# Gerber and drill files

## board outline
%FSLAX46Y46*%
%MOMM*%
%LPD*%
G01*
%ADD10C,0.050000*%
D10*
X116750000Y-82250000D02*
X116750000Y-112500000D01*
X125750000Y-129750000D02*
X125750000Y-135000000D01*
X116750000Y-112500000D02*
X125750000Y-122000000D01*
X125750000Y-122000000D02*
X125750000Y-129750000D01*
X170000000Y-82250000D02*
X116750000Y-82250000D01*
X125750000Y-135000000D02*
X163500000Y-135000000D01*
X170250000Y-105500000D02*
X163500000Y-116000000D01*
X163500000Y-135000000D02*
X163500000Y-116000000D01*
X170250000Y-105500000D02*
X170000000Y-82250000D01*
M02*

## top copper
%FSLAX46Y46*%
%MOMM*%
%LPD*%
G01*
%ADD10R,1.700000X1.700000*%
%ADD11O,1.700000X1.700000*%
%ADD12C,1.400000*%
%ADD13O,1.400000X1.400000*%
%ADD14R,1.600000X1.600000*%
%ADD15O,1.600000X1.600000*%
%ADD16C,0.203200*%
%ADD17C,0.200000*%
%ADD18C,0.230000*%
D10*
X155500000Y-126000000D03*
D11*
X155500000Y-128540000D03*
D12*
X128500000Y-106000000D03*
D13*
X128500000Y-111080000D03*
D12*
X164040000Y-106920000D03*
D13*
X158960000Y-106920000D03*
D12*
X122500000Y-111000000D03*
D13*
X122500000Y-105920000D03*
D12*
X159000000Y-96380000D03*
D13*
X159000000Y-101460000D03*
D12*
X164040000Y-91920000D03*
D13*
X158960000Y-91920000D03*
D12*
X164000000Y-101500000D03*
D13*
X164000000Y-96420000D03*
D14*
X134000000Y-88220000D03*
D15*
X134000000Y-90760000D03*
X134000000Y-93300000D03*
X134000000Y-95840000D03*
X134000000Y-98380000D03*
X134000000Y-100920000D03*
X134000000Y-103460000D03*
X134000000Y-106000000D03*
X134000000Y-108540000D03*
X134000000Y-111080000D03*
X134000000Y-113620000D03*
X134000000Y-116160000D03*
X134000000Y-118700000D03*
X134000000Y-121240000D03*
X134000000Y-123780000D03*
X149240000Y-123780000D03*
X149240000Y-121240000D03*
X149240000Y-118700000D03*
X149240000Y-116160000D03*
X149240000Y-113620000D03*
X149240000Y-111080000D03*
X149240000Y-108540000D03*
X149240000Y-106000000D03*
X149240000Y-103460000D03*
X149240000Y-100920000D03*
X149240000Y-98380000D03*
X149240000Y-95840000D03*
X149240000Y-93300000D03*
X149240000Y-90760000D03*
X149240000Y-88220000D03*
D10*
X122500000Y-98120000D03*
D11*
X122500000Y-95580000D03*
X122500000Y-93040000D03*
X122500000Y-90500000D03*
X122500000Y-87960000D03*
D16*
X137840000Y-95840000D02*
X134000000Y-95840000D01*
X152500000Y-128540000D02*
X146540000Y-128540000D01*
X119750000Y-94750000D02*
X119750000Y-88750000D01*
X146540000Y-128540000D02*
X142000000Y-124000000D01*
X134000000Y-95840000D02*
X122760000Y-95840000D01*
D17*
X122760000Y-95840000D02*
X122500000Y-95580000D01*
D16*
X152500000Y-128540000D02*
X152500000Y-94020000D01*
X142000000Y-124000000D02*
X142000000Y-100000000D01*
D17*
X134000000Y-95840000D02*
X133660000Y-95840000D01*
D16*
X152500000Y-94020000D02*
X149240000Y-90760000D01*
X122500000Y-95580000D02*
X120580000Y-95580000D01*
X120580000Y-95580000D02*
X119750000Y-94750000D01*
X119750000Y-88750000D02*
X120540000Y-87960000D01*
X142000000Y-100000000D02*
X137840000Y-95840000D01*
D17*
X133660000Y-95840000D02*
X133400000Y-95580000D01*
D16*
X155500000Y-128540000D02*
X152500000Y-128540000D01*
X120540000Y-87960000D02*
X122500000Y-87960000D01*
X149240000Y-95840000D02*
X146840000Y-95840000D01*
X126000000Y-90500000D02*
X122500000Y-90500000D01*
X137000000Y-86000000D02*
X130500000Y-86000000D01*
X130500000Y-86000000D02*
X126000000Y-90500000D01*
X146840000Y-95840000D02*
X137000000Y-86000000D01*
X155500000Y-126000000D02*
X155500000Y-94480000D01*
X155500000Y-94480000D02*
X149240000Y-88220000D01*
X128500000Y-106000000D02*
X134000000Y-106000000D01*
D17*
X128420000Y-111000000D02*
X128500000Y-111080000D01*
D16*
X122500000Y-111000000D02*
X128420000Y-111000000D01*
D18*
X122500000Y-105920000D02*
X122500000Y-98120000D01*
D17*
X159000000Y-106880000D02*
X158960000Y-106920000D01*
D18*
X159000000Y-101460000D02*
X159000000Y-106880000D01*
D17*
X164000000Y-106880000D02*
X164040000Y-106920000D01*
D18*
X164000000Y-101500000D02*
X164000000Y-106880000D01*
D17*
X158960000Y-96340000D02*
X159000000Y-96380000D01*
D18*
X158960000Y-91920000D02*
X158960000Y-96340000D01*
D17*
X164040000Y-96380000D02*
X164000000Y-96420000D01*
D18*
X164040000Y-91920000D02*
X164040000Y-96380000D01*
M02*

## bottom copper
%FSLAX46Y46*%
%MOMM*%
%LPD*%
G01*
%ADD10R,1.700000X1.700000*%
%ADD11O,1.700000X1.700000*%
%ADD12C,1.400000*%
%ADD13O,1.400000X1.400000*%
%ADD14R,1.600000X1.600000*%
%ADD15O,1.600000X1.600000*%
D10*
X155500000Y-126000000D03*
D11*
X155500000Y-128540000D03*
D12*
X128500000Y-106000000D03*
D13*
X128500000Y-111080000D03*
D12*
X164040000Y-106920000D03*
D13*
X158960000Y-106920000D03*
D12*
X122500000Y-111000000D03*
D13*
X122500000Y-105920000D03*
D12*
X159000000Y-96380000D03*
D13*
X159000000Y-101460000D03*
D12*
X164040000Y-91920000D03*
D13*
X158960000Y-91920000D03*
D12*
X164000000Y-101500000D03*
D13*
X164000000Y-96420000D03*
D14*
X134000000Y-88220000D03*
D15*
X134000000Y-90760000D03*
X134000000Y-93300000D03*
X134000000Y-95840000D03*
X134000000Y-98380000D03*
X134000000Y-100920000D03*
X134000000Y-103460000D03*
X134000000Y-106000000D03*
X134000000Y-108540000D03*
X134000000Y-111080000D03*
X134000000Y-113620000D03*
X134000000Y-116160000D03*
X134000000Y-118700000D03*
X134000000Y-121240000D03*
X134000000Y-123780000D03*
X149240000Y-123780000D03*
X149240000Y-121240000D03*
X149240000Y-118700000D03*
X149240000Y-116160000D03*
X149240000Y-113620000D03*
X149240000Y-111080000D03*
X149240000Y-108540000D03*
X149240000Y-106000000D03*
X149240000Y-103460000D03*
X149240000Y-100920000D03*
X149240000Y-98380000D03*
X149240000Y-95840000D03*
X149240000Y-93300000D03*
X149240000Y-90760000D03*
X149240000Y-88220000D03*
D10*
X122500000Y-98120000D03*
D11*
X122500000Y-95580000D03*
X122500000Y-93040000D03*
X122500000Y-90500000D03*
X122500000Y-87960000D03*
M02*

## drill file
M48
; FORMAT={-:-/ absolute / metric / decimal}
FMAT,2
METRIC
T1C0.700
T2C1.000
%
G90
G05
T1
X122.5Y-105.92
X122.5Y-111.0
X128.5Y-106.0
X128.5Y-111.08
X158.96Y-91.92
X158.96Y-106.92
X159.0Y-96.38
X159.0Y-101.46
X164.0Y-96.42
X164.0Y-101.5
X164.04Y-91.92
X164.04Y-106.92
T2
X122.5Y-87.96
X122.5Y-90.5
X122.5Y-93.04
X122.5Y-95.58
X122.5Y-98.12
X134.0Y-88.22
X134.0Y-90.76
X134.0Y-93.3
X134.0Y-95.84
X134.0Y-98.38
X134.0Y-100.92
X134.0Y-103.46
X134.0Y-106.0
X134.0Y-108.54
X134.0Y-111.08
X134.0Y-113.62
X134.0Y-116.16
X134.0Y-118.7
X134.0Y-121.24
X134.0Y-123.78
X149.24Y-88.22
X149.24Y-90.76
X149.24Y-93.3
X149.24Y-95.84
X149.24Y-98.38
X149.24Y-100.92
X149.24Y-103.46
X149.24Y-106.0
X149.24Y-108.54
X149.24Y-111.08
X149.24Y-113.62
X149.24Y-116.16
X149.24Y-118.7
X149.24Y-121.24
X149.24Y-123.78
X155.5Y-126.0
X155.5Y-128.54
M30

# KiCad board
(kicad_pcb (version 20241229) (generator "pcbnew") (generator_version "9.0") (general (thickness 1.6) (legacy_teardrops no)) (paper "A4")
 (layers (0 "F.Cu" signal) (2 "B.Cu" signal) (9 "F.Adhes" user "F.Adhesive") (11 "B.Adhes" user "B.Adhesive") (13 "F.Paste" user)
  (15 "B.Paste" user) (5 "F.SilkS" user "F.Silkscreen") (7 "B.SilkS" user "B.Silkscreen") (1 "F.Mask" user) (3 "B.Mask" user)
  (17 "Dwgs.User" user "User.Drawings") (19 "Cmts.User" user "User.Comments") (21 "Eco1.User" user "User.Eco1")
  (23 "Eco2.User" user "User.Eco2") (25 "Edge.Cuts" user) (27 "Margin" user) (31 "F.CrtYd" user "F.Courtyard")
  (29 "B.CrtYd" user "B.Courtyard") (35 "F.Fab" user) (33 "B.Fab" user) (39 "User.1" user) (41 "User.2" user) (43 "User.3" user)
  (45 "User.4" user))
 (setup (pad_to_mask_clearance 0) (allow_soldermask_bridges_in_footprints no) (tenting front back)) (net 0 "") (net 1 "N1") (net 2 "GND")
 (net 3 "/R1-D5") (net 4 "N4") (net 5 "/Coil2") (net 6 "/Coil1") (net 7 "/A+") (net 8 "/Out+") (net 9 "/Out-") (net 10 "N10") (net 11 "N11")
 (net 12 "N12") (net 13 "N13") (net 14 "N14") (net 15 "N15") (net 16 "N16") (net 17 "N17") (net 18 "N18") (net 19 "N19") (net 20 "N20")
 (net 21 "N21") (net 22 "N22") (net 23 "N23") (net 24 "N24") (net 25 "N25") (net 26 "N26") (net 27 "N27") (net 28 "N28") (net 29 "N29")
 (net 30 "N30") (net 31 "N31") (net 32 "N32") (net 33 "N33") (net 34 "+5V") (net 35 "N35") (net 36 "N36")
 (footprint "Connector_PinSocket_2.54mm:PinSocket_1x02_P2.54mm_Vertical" (layer "F.Cu") (at 155.5 126)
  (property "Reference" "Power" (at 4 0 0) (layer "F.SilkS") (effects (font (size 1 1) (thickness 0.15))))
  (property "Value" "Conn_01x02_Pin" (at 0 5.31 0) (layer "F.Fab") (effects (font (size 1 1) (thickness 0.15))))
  (pad "1" thru_hole rect (at 0 0) (size 1.7 1.7) (drill 1) (layers "*.Cu" "*.Mask") (remove_unused_layers no) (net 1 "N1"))
  (pad "2" thru_hole oval (at 0 2.54) (size 1.7 1.7) (drill 1) (layers "*.Cu" "*.Mask") (remove_unused_layers no) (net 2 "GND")))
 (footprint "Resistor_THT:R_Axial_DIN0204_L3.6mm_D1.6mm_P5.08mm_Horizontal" (layer "F.Cu") (at 128.5 106 -90)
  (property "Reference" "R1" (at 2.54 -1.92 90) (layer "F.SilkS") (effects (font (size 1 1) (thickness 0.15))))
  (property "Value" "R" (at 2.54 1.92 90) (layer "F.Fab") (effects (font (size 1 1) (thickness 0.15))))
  (pad "1" thru_hole circle (at 0 0 270) (size 1.4 1.4) (drill 0.7) (layers "*.Cu" "*.Mask") (remove_unused_layers no) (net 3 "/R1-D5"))
  (pad "2" thru_hole oval (at 5.08 0 270) (size 1.4 1.4) (drill 0.7) (layers "*.Cu" "*.Mask") (remove_unused_layers no) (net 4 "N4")))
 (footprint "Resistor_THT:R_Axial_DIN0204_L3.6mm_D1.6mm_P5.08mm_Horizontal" (layer "F.Cu") (at 164.04 106.92 180)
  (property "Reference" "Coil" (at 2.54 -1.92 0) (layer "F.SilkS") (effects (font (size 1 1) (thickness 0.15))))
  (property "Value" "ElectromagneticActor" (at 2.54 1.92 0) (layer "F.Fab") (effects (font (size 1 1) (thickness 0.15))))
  (pad "1" thru_hole circle (at 0 0 180) (size 1.4 1.4) (drill 0.7) (layers "*.Cu" "*.Mask") (remove_unused_layers no) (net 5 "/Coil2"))
  (pad "2" thru_hole oval (at 5.08 0 180) (size 1.4 1.4) (drill 0.7) (layers "*.Cu" "*.Mask") (remove_unused_layers no) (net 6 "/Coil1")))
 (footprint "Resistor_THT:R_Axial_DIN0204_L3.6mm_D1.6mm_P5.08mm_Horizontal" (layer "F.Cu") (at 122.5 111 90)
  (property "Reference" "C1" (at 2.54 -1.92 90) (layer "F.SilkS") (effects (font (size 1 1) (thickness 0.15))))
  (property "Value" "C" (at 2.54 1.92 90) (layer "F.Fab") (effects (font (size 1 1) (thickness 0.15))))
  (pad "1" thru_hole circle (at 0 0 90) (size 1.4 1.4) (drill 0.7) (layers "*.Cu" "*.Mask") (remove_unused_layers no) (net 4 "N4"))
  (pad "2" thru_hole oval (at 5.08 0 90) (size 1.4 1.4) (drill 0.7) (layers "*.Cu" "*.Mask") (remove_unused_layers no) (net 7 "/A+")))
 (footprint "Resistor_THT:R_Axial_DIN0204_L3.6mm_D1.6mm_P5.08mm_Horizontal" (layer "F.Cu") (at 159 96.38 -90)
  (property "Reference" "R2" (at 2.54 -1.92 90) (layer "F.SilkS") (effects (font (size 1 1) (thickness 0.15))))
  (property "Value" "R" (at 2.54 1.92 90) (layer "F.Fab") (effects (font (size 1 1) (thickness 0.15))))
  (pad "1" thru_hole circle (at 0 0 270) (size 1.4 1.4) (drill 0.7) (layers "*.Cu" "*.Mask") (remove_unused_layers no) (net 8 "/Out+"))
  (pad "2" thru_hole oval (at 5.08 0 270) (size 1.4 1.4) (drill 0.7) (layers "*.Cu" "*.Mask") (remove_unused_layers no) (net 6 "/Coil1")))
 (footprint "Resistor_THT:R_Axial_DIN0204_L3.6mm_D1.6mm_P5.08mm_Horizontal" (layer "F.Cu") (at 164.04 91.92 180)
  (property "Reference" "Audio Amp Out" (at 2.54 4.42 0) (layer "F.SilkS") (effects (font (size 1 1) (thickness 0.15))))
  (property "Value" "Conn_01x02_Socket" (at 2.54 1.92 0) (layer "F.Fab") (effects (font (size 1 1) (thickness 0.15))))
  (pad "1" thru_hole circle (at 0 0 180) (size 1.4 1.4) (drill 0.7) (layers "*.Cu" "*.Mask") (remove_unused_layers no) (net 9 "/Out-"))
  (pad "2" thru_hole oval (at 5.08 0 180) (size 1.4 1.4) (drill 0.7) (layers "*.Cu" "*.Mask") (remove_unused_layers no) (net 8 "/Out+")))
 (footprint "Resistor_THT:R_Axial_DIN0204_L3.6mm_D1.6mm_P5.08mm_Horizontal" (layer "F.Cu") (at 164 101.5 90)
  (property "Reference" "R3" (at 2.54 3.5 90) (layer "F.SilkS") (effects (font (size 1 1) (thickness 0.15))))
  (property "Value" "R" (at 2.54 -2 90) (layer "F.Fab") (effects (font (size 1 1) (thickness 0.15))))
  (pad "1" thru_hole circle (at 0 0 90) (size 1.4 1.4) (drill 0.7) (layers "*.Cu" "*.Mask") (remove_unused_layers no) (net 5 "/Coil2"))
  (pad "2" thru_hole oval (at 5.08 0 90) (size 1.4 1.4) (drill 0.7) (layers "*.Cu" "*.Mask") (remove_unused_layers no) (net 9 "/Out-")))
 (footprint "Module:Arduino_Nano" (layer "F.Cu") (at 134 88.22)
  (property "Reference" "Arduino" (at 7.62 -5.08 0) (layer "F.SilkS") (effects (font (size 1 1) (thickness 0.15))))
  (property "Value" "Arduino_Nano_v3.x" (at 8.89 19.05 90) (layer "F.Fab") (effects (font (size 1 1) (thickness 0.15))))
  (pad "1" thru_hole rect (at 0 0) (size 1.6 1.6) (drill 1) (layers "*.Cu" "*.Mask") (remove_unused_layers no) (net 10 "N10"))
  (pad "2" thru_hole oval (at 0 2.54) (size 1.6 1.6) (drill 1) (layers "*.Cu" "*.Mask") (remove_unused_layers no) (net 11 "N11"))
  (pad "3" thru_hole oval (at 0 5.08) (size 1.6 1.6) (drill 1) (layers "*.Cu" "*.Mask") (remove_unused_layers no) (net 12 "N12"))
  (pad "4" thru_hole oval (at 0 7.62) (size 1.6 1.6) (drill 1) (layers "*.Cu" "*.Mask") (remove_unused_layers no) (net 2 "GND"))
  (pad "5" thru_hole oval (at 0 10.16) (size 1.6 1.6) (drill 1) (layers "*.Cu" "*.Mask") (remove_unused_layers no) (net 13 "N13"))
  (pad "6" thru_hole oval (at 0 12.7) (size 1.6 1.6) (drill 1) (layers "*.Cu" "*.Mask") (remove_unused_layers no) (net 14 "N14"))
  (pad "7" thru_hole oval (at 0 15.24) (size 1.6 1.6) (drill 1) (layers "*.Cu" "*.Mask") (remove_unused_layers no) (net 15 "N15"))
  (pad "8" thru_hole oval (at 0 17.78) (size 1.6 1.6) (drill 1) (layers "*.Cu" "*.Mask") (remove_unused_layers no) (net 3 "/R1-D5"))
  (pad "9" thru_hole oval (at 0 20.32) (size 1.6 1.6) (drill 1) (layers "*.Cu" "*.Mask") (remove_unused_layers no) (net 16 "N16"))
  (pad "10" thru_hole oval (at 0 22.86) (size 1.6 1.6) (drill 1) (layers "*.Cu" "*.Mask") (remove_unused_layers no) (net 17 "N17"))
  (pad "11" thru_hole oval (at 0 25.4) (size 1.6 1.6) (drill 1) (layers "*.Cu" "*.Mask") (remove_unused_layers no) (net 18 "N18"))
  (pad "12" thru_hole oval (at 0 27.94) (size 1.6 1.6) (drill 1) (layers "*.Cu" "*.Mask") (remove_unused_layers no) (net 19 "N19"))
  (pad "13" thru_hole oval (at 0 30.48) (size 1.6 1.6) (drill 1) (layers "*.Cu" "*.Mask") (remove_unused_layers no) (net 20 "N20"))
  (pad "14" thru_hole oval (at 0 33.02) (size 1.6 1.6) (drill 1) (layers "*.Cu" "*.Mask") (remove_unused_layers no) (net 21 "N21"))
  (pad "15" thru_hole oval (at 0 35.56) (size 1.6 1.6) (drill 1) (layers "*.Cu" "*.Mask") (remove_unused_layers no) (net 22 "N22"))
  (pad "16" thru_hole oval (at 15.24 35.56) (size 1.6 1.6) (drill 1) (layers "*.Cu" "*.Mask") (remove_unused_layers no) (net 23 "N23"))
  (pad "17" thru_hole oval (at 15.24 33.02) (size 1.6 1.6) (drill 1) (layers "*.Cu" "*.Mask") (remove_unused_layers no) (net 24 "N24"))
  (pad "18" thru_hole oval (at 15.24 30.48) (size 1.6 1.6) (drill 1) (layers "*.Cu" "*.Mask") (remove_unused_layers no) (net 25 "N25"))
  (pad "19" thru_hole oval (at 15.24 27.94) (size 1.6 1.6) (drill 1) (layers "*.Cu" "*.Mask") (remove_unused_layers no) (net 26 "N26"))
  (pad "20" thru_hole oval (at 15.24 25.4) (size 1.6 1.6) (drill 1) (layers "*.Cu" "*.Mask") (remove_unused_layers no) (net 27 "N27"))
  (pad "21" thru_hole oval (at 15.24 22.86) (size 1.6 1.6) (drill 1) (layers "*.Cu" "*.Mask") (remove_unused_layers no) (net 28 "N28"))
  (pad "22" thru_hole oval (at 15.24 20.32) (size 1.6 1.6) (drill 1) (layers "*.Cu" "*.Mask") (remove_unused_layers no) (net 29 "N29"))
  (pad "23" thru_hole oval (at 15.24 17.78) (size 1.6 1.6) (drill 1) (layers "*.Cu" "*.Mask") (remove_unused_layers no) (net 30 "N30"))
  (pad "24" thru_hole oval (at 15.24 15.24) (size 1.6 1.6) (drill 1) (layers "*.Cu" "*.Mask") (remove_unused_layers no) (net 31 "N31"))
  (pad "25" thru_hole oval (at 15.24 12.7) (size 1.6 1.6) (drill 1) (layers "*.Cu" "*.Mask") (remove_unused_layers no) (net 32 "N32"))
  (pad "26" thru_hole oval (at 15.24 10.16) (size 1.6 1.6) (drill 1) (layers "*.Cu" "*.Mask") (remove_unused_layers no) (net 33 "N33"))
  (pad "27" thru_hole oval (at 15.24 7.62) (size 1.6 1.6) (drill 1) (layers "*.Cu" "*.Mask") (remove_unused_layers no) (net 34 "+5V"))
  (pad "28" thru_hole oval (at 15.24 5.08) (size 1.6 1.6) (drill 1) (layers "*.Cu" "*.Mask") (remove_unused_layers no) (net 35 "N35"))
  (pad "29" thru_hole oval (at 15.24 2.54) (size 1.6 1.6) (drill 1) (layers "*.Cu" "*.Mask") (remove_unused_layers no) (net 2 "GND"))
  (pad "30" thru_hole oval (at 15.24 0) (size 1.6 1.6) (drill 1) (layers "*.Cu" "*.Mask") (remove_unused_layers no) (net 1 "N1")))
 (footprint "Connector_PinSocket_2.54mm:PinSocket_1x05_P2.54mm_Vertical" (layer "F.Cu") (at 122.5 98.12 180)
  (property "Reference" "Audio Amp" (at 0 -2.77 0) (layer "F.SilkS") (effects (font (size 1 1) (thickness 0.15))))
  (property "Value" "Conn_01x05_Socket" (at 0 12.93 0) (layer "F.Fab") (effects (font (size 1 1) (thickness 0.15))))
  (pad "1" thru_hole rect (at 0 0 180) (size 1.7 1.7) (drill 1) (layers "*.Cu" "*.Mask") (remove_unused_layers no) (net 7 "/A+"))
  (pad "2" thru_hole oval (at 0 2.54 180) (size 1.7 1.7) (drill 1) (layers "*.Cu" "*.Mask") (remove_unused_layers no) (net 2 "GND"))
  (pad "3" thru_hole oval (at 0 5.08 180) (size 1.7 1.7) (drill 1) (layers "*.Cu" "*.Mask") (remove_unused_layers no) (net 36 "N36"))
  (pad "4" thru_hole oval (at 0 7.62 180) (size 1.7 1.7) (drill 1) (layers "*.Cu" "*.Mask") (remove_unused_layers no) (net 34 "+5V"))
  (pad "5" thru_hole oval (at 0 10.16 180) (size 1.7 1.7) (drill 1) (layers "*.Cu" "*.Mask") (remove_unused_layers no) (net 2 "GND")))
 (gr_line (start 116.75 82.25) (end 116.75 112.5) (stroke (width 0.05) (type default)) (layer "Edge.Cuts"))
 (gr_line (start 125.75 129.75) (end 125.75 135) (stroke (width 0.05) (type default)) (layer "Edge.Cuts"))
 (gr_line (start 116.75 112.5) (end 125.75 122) (stroke (width 0.05) (type default)) (layer "Edge.Cuts"))
 (gr_line (start 125.75 122) (end 125.75 129.75) (stroke (width 0.05) (type default)) (layer "Edge.Cuts"))
 (gr_line (start 170 82.25) (end 116.75 82.25) (stroke (width 0.05) (type default)) (layer "Edge.Cuts"))
 (gr_line (start 125.75 135) (end 163.5 135) (stroke (width 0.05) (type default)) (layer "Edge.Cuts"))
 (gr_line (start 170.25 105.5) (end 163.5 116) (stroke (width 0.05) (type default)) (layer "Edge.Cuts"))
 (gr_line (start 163.5 135) (end 163.5 116) (stroke (width 0.05) (type default)) (layer "Edge.Cuts"))
 (gr_line (start 170.25 105.5) (end 170 82.25) (stroke (width 0.05) (type default)) (layer "Edge.Cuts"))
 (segment (start 137.84 95.84) (end 134 95.84) (width 0.2032) (layer "F.Cu") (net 2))
 (segment (start 152.5 128.54) (end 146.54 128.54) (width 0.2032) (layer "F.Cu") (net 2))
 (segment (start 119.75 94.75) (end 119.75 88.75) (width 0.2032) (layer "F.Cu") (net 2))
 (segment (start 146.54 128.54) (end 142 124) (width 0.2032) (layer "F.Cu") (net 2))
 (segment (start 134 95.84) (end 122.76 95.84) (width 0.2032) (layer "F.Cu") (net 2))
 (segment (start 122.76 95.84) (end 122.5 95.58) (width 0.2) (layer "F.Cu") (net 2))
 (segment (start 152.5 128.54) (end 152.5 94.02) (width 0.2032) (layer "F.Cu") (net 2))
 (segment (start 142 124) (end 142 100) (width 0.2032) (layer "F.Cu") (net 2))
 (segment (start 134 95.84) (end 133.66 95.84) (width 0.2) (layer "F.Cu") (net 2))
 (segment (start 152.5 94.02) (end 149.24 90.76) (width 0.2032) (layer "F.Cu") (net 2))
 (segment (start 122.5 95.58) (end 120.58 95.58) (width 0.2032) (layer "F.Cu") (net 2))
 (segment (start 120.58 95.58) (end 119.75 94.75) (width 0.2032) (layer "F.Cu") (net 2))
 (segment (start 119.75 88.75) (end 120.54 87.96) (width 0.2032) (layer "F.Cu") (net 2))
 (segment (start 142 100) (end 137.84 95.84) (width 0.2032) (layer "F.Cu") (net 2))
 (segment (start 133.66 95.84) (end 133.4 95.58) (width 0.2) (layer "F.Cu") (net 2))
 (segment (start 155.5 128.54) (end 152.5 128.54) (width 0.2032) (layer "F.Cu") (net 2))
 (segment (start 120.54 87.96) (end 122.5 87.96) (width 0.2032) (layer "F.Cu") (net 2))
 (segment (start 149.24 95.84) (end 146.84 95.84) (width 0.2032) (layer "F.Cu") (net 34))
 (segment (start 126 90.5) (end 122.5 90.5) (width 0.2032) (layer "F.Cu") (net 34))
 (segment (start 137 86) (end 130.5 86) (width 0.2032) (layer "F.Cu") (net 34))
 (segment (start 130.5 86) (end 126 90.5) (width 0.2032) (layer "F.Cu") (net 34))
 (segment (start 146.84 95.84) (end 137 86) (width 0.2032) (layer "F.Cu") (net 34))
 (segment (start 155.5 126) (end 155.5 94.48) (width 0.2032) (layer "F.Cu") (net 1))
 (segment (start 155.5 94.48) (end 149.24 88.22) (width 0.2032) (layer "F.Cu") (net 1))
 (segment (start 128.5 106) (end 134 106) (width 0.2032) (layer "F.Cu") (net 3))
 (segment (start 128.42 111) (end 128.5 111.08) (width 0.2) (layer "F.Cu") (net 4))
 (segment (start 122.5 111) (end 128.42 111) (width 0.2032) (layer "F.Cu") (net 4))
 (segment (start 122.5 105.92) (end 122.5 98.12) (width 0.23) (layer "F.Cu") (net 7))
 (segment (start 159 106.88) (end 158.96 106.92) (width 0.2) (layer "F.Cu") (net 6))
 (segment (start 159 101.46) (end 159 106.88) (width 0.23) (layer "F.Cu") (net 6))
 (segment (start 164 106.88) (end 164.04 106.92) (width 0.2) (layer "F.Cu") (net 5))
 (segment (start 164 101.5) (end 164 106.88) (width 0.23) (layer "F.Cu") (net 5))
 (segment (start 158.96 96.34) (end 159 96.38) (width 0.2) (layer "F.Cu") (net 8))
 (segment (start 158.96 91.92) (end 158.96 96.34) (width 0.23) (layer "F.Cu") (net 8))
 (segment (start 164.04 96.38) (end 164 96.42) (width 0.2) (layer "F.Cu") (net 9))
 (segment (start 164.04 91.92) (end 164.04 96.38) (width 0.23) (layer "F.Cu") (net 9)))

